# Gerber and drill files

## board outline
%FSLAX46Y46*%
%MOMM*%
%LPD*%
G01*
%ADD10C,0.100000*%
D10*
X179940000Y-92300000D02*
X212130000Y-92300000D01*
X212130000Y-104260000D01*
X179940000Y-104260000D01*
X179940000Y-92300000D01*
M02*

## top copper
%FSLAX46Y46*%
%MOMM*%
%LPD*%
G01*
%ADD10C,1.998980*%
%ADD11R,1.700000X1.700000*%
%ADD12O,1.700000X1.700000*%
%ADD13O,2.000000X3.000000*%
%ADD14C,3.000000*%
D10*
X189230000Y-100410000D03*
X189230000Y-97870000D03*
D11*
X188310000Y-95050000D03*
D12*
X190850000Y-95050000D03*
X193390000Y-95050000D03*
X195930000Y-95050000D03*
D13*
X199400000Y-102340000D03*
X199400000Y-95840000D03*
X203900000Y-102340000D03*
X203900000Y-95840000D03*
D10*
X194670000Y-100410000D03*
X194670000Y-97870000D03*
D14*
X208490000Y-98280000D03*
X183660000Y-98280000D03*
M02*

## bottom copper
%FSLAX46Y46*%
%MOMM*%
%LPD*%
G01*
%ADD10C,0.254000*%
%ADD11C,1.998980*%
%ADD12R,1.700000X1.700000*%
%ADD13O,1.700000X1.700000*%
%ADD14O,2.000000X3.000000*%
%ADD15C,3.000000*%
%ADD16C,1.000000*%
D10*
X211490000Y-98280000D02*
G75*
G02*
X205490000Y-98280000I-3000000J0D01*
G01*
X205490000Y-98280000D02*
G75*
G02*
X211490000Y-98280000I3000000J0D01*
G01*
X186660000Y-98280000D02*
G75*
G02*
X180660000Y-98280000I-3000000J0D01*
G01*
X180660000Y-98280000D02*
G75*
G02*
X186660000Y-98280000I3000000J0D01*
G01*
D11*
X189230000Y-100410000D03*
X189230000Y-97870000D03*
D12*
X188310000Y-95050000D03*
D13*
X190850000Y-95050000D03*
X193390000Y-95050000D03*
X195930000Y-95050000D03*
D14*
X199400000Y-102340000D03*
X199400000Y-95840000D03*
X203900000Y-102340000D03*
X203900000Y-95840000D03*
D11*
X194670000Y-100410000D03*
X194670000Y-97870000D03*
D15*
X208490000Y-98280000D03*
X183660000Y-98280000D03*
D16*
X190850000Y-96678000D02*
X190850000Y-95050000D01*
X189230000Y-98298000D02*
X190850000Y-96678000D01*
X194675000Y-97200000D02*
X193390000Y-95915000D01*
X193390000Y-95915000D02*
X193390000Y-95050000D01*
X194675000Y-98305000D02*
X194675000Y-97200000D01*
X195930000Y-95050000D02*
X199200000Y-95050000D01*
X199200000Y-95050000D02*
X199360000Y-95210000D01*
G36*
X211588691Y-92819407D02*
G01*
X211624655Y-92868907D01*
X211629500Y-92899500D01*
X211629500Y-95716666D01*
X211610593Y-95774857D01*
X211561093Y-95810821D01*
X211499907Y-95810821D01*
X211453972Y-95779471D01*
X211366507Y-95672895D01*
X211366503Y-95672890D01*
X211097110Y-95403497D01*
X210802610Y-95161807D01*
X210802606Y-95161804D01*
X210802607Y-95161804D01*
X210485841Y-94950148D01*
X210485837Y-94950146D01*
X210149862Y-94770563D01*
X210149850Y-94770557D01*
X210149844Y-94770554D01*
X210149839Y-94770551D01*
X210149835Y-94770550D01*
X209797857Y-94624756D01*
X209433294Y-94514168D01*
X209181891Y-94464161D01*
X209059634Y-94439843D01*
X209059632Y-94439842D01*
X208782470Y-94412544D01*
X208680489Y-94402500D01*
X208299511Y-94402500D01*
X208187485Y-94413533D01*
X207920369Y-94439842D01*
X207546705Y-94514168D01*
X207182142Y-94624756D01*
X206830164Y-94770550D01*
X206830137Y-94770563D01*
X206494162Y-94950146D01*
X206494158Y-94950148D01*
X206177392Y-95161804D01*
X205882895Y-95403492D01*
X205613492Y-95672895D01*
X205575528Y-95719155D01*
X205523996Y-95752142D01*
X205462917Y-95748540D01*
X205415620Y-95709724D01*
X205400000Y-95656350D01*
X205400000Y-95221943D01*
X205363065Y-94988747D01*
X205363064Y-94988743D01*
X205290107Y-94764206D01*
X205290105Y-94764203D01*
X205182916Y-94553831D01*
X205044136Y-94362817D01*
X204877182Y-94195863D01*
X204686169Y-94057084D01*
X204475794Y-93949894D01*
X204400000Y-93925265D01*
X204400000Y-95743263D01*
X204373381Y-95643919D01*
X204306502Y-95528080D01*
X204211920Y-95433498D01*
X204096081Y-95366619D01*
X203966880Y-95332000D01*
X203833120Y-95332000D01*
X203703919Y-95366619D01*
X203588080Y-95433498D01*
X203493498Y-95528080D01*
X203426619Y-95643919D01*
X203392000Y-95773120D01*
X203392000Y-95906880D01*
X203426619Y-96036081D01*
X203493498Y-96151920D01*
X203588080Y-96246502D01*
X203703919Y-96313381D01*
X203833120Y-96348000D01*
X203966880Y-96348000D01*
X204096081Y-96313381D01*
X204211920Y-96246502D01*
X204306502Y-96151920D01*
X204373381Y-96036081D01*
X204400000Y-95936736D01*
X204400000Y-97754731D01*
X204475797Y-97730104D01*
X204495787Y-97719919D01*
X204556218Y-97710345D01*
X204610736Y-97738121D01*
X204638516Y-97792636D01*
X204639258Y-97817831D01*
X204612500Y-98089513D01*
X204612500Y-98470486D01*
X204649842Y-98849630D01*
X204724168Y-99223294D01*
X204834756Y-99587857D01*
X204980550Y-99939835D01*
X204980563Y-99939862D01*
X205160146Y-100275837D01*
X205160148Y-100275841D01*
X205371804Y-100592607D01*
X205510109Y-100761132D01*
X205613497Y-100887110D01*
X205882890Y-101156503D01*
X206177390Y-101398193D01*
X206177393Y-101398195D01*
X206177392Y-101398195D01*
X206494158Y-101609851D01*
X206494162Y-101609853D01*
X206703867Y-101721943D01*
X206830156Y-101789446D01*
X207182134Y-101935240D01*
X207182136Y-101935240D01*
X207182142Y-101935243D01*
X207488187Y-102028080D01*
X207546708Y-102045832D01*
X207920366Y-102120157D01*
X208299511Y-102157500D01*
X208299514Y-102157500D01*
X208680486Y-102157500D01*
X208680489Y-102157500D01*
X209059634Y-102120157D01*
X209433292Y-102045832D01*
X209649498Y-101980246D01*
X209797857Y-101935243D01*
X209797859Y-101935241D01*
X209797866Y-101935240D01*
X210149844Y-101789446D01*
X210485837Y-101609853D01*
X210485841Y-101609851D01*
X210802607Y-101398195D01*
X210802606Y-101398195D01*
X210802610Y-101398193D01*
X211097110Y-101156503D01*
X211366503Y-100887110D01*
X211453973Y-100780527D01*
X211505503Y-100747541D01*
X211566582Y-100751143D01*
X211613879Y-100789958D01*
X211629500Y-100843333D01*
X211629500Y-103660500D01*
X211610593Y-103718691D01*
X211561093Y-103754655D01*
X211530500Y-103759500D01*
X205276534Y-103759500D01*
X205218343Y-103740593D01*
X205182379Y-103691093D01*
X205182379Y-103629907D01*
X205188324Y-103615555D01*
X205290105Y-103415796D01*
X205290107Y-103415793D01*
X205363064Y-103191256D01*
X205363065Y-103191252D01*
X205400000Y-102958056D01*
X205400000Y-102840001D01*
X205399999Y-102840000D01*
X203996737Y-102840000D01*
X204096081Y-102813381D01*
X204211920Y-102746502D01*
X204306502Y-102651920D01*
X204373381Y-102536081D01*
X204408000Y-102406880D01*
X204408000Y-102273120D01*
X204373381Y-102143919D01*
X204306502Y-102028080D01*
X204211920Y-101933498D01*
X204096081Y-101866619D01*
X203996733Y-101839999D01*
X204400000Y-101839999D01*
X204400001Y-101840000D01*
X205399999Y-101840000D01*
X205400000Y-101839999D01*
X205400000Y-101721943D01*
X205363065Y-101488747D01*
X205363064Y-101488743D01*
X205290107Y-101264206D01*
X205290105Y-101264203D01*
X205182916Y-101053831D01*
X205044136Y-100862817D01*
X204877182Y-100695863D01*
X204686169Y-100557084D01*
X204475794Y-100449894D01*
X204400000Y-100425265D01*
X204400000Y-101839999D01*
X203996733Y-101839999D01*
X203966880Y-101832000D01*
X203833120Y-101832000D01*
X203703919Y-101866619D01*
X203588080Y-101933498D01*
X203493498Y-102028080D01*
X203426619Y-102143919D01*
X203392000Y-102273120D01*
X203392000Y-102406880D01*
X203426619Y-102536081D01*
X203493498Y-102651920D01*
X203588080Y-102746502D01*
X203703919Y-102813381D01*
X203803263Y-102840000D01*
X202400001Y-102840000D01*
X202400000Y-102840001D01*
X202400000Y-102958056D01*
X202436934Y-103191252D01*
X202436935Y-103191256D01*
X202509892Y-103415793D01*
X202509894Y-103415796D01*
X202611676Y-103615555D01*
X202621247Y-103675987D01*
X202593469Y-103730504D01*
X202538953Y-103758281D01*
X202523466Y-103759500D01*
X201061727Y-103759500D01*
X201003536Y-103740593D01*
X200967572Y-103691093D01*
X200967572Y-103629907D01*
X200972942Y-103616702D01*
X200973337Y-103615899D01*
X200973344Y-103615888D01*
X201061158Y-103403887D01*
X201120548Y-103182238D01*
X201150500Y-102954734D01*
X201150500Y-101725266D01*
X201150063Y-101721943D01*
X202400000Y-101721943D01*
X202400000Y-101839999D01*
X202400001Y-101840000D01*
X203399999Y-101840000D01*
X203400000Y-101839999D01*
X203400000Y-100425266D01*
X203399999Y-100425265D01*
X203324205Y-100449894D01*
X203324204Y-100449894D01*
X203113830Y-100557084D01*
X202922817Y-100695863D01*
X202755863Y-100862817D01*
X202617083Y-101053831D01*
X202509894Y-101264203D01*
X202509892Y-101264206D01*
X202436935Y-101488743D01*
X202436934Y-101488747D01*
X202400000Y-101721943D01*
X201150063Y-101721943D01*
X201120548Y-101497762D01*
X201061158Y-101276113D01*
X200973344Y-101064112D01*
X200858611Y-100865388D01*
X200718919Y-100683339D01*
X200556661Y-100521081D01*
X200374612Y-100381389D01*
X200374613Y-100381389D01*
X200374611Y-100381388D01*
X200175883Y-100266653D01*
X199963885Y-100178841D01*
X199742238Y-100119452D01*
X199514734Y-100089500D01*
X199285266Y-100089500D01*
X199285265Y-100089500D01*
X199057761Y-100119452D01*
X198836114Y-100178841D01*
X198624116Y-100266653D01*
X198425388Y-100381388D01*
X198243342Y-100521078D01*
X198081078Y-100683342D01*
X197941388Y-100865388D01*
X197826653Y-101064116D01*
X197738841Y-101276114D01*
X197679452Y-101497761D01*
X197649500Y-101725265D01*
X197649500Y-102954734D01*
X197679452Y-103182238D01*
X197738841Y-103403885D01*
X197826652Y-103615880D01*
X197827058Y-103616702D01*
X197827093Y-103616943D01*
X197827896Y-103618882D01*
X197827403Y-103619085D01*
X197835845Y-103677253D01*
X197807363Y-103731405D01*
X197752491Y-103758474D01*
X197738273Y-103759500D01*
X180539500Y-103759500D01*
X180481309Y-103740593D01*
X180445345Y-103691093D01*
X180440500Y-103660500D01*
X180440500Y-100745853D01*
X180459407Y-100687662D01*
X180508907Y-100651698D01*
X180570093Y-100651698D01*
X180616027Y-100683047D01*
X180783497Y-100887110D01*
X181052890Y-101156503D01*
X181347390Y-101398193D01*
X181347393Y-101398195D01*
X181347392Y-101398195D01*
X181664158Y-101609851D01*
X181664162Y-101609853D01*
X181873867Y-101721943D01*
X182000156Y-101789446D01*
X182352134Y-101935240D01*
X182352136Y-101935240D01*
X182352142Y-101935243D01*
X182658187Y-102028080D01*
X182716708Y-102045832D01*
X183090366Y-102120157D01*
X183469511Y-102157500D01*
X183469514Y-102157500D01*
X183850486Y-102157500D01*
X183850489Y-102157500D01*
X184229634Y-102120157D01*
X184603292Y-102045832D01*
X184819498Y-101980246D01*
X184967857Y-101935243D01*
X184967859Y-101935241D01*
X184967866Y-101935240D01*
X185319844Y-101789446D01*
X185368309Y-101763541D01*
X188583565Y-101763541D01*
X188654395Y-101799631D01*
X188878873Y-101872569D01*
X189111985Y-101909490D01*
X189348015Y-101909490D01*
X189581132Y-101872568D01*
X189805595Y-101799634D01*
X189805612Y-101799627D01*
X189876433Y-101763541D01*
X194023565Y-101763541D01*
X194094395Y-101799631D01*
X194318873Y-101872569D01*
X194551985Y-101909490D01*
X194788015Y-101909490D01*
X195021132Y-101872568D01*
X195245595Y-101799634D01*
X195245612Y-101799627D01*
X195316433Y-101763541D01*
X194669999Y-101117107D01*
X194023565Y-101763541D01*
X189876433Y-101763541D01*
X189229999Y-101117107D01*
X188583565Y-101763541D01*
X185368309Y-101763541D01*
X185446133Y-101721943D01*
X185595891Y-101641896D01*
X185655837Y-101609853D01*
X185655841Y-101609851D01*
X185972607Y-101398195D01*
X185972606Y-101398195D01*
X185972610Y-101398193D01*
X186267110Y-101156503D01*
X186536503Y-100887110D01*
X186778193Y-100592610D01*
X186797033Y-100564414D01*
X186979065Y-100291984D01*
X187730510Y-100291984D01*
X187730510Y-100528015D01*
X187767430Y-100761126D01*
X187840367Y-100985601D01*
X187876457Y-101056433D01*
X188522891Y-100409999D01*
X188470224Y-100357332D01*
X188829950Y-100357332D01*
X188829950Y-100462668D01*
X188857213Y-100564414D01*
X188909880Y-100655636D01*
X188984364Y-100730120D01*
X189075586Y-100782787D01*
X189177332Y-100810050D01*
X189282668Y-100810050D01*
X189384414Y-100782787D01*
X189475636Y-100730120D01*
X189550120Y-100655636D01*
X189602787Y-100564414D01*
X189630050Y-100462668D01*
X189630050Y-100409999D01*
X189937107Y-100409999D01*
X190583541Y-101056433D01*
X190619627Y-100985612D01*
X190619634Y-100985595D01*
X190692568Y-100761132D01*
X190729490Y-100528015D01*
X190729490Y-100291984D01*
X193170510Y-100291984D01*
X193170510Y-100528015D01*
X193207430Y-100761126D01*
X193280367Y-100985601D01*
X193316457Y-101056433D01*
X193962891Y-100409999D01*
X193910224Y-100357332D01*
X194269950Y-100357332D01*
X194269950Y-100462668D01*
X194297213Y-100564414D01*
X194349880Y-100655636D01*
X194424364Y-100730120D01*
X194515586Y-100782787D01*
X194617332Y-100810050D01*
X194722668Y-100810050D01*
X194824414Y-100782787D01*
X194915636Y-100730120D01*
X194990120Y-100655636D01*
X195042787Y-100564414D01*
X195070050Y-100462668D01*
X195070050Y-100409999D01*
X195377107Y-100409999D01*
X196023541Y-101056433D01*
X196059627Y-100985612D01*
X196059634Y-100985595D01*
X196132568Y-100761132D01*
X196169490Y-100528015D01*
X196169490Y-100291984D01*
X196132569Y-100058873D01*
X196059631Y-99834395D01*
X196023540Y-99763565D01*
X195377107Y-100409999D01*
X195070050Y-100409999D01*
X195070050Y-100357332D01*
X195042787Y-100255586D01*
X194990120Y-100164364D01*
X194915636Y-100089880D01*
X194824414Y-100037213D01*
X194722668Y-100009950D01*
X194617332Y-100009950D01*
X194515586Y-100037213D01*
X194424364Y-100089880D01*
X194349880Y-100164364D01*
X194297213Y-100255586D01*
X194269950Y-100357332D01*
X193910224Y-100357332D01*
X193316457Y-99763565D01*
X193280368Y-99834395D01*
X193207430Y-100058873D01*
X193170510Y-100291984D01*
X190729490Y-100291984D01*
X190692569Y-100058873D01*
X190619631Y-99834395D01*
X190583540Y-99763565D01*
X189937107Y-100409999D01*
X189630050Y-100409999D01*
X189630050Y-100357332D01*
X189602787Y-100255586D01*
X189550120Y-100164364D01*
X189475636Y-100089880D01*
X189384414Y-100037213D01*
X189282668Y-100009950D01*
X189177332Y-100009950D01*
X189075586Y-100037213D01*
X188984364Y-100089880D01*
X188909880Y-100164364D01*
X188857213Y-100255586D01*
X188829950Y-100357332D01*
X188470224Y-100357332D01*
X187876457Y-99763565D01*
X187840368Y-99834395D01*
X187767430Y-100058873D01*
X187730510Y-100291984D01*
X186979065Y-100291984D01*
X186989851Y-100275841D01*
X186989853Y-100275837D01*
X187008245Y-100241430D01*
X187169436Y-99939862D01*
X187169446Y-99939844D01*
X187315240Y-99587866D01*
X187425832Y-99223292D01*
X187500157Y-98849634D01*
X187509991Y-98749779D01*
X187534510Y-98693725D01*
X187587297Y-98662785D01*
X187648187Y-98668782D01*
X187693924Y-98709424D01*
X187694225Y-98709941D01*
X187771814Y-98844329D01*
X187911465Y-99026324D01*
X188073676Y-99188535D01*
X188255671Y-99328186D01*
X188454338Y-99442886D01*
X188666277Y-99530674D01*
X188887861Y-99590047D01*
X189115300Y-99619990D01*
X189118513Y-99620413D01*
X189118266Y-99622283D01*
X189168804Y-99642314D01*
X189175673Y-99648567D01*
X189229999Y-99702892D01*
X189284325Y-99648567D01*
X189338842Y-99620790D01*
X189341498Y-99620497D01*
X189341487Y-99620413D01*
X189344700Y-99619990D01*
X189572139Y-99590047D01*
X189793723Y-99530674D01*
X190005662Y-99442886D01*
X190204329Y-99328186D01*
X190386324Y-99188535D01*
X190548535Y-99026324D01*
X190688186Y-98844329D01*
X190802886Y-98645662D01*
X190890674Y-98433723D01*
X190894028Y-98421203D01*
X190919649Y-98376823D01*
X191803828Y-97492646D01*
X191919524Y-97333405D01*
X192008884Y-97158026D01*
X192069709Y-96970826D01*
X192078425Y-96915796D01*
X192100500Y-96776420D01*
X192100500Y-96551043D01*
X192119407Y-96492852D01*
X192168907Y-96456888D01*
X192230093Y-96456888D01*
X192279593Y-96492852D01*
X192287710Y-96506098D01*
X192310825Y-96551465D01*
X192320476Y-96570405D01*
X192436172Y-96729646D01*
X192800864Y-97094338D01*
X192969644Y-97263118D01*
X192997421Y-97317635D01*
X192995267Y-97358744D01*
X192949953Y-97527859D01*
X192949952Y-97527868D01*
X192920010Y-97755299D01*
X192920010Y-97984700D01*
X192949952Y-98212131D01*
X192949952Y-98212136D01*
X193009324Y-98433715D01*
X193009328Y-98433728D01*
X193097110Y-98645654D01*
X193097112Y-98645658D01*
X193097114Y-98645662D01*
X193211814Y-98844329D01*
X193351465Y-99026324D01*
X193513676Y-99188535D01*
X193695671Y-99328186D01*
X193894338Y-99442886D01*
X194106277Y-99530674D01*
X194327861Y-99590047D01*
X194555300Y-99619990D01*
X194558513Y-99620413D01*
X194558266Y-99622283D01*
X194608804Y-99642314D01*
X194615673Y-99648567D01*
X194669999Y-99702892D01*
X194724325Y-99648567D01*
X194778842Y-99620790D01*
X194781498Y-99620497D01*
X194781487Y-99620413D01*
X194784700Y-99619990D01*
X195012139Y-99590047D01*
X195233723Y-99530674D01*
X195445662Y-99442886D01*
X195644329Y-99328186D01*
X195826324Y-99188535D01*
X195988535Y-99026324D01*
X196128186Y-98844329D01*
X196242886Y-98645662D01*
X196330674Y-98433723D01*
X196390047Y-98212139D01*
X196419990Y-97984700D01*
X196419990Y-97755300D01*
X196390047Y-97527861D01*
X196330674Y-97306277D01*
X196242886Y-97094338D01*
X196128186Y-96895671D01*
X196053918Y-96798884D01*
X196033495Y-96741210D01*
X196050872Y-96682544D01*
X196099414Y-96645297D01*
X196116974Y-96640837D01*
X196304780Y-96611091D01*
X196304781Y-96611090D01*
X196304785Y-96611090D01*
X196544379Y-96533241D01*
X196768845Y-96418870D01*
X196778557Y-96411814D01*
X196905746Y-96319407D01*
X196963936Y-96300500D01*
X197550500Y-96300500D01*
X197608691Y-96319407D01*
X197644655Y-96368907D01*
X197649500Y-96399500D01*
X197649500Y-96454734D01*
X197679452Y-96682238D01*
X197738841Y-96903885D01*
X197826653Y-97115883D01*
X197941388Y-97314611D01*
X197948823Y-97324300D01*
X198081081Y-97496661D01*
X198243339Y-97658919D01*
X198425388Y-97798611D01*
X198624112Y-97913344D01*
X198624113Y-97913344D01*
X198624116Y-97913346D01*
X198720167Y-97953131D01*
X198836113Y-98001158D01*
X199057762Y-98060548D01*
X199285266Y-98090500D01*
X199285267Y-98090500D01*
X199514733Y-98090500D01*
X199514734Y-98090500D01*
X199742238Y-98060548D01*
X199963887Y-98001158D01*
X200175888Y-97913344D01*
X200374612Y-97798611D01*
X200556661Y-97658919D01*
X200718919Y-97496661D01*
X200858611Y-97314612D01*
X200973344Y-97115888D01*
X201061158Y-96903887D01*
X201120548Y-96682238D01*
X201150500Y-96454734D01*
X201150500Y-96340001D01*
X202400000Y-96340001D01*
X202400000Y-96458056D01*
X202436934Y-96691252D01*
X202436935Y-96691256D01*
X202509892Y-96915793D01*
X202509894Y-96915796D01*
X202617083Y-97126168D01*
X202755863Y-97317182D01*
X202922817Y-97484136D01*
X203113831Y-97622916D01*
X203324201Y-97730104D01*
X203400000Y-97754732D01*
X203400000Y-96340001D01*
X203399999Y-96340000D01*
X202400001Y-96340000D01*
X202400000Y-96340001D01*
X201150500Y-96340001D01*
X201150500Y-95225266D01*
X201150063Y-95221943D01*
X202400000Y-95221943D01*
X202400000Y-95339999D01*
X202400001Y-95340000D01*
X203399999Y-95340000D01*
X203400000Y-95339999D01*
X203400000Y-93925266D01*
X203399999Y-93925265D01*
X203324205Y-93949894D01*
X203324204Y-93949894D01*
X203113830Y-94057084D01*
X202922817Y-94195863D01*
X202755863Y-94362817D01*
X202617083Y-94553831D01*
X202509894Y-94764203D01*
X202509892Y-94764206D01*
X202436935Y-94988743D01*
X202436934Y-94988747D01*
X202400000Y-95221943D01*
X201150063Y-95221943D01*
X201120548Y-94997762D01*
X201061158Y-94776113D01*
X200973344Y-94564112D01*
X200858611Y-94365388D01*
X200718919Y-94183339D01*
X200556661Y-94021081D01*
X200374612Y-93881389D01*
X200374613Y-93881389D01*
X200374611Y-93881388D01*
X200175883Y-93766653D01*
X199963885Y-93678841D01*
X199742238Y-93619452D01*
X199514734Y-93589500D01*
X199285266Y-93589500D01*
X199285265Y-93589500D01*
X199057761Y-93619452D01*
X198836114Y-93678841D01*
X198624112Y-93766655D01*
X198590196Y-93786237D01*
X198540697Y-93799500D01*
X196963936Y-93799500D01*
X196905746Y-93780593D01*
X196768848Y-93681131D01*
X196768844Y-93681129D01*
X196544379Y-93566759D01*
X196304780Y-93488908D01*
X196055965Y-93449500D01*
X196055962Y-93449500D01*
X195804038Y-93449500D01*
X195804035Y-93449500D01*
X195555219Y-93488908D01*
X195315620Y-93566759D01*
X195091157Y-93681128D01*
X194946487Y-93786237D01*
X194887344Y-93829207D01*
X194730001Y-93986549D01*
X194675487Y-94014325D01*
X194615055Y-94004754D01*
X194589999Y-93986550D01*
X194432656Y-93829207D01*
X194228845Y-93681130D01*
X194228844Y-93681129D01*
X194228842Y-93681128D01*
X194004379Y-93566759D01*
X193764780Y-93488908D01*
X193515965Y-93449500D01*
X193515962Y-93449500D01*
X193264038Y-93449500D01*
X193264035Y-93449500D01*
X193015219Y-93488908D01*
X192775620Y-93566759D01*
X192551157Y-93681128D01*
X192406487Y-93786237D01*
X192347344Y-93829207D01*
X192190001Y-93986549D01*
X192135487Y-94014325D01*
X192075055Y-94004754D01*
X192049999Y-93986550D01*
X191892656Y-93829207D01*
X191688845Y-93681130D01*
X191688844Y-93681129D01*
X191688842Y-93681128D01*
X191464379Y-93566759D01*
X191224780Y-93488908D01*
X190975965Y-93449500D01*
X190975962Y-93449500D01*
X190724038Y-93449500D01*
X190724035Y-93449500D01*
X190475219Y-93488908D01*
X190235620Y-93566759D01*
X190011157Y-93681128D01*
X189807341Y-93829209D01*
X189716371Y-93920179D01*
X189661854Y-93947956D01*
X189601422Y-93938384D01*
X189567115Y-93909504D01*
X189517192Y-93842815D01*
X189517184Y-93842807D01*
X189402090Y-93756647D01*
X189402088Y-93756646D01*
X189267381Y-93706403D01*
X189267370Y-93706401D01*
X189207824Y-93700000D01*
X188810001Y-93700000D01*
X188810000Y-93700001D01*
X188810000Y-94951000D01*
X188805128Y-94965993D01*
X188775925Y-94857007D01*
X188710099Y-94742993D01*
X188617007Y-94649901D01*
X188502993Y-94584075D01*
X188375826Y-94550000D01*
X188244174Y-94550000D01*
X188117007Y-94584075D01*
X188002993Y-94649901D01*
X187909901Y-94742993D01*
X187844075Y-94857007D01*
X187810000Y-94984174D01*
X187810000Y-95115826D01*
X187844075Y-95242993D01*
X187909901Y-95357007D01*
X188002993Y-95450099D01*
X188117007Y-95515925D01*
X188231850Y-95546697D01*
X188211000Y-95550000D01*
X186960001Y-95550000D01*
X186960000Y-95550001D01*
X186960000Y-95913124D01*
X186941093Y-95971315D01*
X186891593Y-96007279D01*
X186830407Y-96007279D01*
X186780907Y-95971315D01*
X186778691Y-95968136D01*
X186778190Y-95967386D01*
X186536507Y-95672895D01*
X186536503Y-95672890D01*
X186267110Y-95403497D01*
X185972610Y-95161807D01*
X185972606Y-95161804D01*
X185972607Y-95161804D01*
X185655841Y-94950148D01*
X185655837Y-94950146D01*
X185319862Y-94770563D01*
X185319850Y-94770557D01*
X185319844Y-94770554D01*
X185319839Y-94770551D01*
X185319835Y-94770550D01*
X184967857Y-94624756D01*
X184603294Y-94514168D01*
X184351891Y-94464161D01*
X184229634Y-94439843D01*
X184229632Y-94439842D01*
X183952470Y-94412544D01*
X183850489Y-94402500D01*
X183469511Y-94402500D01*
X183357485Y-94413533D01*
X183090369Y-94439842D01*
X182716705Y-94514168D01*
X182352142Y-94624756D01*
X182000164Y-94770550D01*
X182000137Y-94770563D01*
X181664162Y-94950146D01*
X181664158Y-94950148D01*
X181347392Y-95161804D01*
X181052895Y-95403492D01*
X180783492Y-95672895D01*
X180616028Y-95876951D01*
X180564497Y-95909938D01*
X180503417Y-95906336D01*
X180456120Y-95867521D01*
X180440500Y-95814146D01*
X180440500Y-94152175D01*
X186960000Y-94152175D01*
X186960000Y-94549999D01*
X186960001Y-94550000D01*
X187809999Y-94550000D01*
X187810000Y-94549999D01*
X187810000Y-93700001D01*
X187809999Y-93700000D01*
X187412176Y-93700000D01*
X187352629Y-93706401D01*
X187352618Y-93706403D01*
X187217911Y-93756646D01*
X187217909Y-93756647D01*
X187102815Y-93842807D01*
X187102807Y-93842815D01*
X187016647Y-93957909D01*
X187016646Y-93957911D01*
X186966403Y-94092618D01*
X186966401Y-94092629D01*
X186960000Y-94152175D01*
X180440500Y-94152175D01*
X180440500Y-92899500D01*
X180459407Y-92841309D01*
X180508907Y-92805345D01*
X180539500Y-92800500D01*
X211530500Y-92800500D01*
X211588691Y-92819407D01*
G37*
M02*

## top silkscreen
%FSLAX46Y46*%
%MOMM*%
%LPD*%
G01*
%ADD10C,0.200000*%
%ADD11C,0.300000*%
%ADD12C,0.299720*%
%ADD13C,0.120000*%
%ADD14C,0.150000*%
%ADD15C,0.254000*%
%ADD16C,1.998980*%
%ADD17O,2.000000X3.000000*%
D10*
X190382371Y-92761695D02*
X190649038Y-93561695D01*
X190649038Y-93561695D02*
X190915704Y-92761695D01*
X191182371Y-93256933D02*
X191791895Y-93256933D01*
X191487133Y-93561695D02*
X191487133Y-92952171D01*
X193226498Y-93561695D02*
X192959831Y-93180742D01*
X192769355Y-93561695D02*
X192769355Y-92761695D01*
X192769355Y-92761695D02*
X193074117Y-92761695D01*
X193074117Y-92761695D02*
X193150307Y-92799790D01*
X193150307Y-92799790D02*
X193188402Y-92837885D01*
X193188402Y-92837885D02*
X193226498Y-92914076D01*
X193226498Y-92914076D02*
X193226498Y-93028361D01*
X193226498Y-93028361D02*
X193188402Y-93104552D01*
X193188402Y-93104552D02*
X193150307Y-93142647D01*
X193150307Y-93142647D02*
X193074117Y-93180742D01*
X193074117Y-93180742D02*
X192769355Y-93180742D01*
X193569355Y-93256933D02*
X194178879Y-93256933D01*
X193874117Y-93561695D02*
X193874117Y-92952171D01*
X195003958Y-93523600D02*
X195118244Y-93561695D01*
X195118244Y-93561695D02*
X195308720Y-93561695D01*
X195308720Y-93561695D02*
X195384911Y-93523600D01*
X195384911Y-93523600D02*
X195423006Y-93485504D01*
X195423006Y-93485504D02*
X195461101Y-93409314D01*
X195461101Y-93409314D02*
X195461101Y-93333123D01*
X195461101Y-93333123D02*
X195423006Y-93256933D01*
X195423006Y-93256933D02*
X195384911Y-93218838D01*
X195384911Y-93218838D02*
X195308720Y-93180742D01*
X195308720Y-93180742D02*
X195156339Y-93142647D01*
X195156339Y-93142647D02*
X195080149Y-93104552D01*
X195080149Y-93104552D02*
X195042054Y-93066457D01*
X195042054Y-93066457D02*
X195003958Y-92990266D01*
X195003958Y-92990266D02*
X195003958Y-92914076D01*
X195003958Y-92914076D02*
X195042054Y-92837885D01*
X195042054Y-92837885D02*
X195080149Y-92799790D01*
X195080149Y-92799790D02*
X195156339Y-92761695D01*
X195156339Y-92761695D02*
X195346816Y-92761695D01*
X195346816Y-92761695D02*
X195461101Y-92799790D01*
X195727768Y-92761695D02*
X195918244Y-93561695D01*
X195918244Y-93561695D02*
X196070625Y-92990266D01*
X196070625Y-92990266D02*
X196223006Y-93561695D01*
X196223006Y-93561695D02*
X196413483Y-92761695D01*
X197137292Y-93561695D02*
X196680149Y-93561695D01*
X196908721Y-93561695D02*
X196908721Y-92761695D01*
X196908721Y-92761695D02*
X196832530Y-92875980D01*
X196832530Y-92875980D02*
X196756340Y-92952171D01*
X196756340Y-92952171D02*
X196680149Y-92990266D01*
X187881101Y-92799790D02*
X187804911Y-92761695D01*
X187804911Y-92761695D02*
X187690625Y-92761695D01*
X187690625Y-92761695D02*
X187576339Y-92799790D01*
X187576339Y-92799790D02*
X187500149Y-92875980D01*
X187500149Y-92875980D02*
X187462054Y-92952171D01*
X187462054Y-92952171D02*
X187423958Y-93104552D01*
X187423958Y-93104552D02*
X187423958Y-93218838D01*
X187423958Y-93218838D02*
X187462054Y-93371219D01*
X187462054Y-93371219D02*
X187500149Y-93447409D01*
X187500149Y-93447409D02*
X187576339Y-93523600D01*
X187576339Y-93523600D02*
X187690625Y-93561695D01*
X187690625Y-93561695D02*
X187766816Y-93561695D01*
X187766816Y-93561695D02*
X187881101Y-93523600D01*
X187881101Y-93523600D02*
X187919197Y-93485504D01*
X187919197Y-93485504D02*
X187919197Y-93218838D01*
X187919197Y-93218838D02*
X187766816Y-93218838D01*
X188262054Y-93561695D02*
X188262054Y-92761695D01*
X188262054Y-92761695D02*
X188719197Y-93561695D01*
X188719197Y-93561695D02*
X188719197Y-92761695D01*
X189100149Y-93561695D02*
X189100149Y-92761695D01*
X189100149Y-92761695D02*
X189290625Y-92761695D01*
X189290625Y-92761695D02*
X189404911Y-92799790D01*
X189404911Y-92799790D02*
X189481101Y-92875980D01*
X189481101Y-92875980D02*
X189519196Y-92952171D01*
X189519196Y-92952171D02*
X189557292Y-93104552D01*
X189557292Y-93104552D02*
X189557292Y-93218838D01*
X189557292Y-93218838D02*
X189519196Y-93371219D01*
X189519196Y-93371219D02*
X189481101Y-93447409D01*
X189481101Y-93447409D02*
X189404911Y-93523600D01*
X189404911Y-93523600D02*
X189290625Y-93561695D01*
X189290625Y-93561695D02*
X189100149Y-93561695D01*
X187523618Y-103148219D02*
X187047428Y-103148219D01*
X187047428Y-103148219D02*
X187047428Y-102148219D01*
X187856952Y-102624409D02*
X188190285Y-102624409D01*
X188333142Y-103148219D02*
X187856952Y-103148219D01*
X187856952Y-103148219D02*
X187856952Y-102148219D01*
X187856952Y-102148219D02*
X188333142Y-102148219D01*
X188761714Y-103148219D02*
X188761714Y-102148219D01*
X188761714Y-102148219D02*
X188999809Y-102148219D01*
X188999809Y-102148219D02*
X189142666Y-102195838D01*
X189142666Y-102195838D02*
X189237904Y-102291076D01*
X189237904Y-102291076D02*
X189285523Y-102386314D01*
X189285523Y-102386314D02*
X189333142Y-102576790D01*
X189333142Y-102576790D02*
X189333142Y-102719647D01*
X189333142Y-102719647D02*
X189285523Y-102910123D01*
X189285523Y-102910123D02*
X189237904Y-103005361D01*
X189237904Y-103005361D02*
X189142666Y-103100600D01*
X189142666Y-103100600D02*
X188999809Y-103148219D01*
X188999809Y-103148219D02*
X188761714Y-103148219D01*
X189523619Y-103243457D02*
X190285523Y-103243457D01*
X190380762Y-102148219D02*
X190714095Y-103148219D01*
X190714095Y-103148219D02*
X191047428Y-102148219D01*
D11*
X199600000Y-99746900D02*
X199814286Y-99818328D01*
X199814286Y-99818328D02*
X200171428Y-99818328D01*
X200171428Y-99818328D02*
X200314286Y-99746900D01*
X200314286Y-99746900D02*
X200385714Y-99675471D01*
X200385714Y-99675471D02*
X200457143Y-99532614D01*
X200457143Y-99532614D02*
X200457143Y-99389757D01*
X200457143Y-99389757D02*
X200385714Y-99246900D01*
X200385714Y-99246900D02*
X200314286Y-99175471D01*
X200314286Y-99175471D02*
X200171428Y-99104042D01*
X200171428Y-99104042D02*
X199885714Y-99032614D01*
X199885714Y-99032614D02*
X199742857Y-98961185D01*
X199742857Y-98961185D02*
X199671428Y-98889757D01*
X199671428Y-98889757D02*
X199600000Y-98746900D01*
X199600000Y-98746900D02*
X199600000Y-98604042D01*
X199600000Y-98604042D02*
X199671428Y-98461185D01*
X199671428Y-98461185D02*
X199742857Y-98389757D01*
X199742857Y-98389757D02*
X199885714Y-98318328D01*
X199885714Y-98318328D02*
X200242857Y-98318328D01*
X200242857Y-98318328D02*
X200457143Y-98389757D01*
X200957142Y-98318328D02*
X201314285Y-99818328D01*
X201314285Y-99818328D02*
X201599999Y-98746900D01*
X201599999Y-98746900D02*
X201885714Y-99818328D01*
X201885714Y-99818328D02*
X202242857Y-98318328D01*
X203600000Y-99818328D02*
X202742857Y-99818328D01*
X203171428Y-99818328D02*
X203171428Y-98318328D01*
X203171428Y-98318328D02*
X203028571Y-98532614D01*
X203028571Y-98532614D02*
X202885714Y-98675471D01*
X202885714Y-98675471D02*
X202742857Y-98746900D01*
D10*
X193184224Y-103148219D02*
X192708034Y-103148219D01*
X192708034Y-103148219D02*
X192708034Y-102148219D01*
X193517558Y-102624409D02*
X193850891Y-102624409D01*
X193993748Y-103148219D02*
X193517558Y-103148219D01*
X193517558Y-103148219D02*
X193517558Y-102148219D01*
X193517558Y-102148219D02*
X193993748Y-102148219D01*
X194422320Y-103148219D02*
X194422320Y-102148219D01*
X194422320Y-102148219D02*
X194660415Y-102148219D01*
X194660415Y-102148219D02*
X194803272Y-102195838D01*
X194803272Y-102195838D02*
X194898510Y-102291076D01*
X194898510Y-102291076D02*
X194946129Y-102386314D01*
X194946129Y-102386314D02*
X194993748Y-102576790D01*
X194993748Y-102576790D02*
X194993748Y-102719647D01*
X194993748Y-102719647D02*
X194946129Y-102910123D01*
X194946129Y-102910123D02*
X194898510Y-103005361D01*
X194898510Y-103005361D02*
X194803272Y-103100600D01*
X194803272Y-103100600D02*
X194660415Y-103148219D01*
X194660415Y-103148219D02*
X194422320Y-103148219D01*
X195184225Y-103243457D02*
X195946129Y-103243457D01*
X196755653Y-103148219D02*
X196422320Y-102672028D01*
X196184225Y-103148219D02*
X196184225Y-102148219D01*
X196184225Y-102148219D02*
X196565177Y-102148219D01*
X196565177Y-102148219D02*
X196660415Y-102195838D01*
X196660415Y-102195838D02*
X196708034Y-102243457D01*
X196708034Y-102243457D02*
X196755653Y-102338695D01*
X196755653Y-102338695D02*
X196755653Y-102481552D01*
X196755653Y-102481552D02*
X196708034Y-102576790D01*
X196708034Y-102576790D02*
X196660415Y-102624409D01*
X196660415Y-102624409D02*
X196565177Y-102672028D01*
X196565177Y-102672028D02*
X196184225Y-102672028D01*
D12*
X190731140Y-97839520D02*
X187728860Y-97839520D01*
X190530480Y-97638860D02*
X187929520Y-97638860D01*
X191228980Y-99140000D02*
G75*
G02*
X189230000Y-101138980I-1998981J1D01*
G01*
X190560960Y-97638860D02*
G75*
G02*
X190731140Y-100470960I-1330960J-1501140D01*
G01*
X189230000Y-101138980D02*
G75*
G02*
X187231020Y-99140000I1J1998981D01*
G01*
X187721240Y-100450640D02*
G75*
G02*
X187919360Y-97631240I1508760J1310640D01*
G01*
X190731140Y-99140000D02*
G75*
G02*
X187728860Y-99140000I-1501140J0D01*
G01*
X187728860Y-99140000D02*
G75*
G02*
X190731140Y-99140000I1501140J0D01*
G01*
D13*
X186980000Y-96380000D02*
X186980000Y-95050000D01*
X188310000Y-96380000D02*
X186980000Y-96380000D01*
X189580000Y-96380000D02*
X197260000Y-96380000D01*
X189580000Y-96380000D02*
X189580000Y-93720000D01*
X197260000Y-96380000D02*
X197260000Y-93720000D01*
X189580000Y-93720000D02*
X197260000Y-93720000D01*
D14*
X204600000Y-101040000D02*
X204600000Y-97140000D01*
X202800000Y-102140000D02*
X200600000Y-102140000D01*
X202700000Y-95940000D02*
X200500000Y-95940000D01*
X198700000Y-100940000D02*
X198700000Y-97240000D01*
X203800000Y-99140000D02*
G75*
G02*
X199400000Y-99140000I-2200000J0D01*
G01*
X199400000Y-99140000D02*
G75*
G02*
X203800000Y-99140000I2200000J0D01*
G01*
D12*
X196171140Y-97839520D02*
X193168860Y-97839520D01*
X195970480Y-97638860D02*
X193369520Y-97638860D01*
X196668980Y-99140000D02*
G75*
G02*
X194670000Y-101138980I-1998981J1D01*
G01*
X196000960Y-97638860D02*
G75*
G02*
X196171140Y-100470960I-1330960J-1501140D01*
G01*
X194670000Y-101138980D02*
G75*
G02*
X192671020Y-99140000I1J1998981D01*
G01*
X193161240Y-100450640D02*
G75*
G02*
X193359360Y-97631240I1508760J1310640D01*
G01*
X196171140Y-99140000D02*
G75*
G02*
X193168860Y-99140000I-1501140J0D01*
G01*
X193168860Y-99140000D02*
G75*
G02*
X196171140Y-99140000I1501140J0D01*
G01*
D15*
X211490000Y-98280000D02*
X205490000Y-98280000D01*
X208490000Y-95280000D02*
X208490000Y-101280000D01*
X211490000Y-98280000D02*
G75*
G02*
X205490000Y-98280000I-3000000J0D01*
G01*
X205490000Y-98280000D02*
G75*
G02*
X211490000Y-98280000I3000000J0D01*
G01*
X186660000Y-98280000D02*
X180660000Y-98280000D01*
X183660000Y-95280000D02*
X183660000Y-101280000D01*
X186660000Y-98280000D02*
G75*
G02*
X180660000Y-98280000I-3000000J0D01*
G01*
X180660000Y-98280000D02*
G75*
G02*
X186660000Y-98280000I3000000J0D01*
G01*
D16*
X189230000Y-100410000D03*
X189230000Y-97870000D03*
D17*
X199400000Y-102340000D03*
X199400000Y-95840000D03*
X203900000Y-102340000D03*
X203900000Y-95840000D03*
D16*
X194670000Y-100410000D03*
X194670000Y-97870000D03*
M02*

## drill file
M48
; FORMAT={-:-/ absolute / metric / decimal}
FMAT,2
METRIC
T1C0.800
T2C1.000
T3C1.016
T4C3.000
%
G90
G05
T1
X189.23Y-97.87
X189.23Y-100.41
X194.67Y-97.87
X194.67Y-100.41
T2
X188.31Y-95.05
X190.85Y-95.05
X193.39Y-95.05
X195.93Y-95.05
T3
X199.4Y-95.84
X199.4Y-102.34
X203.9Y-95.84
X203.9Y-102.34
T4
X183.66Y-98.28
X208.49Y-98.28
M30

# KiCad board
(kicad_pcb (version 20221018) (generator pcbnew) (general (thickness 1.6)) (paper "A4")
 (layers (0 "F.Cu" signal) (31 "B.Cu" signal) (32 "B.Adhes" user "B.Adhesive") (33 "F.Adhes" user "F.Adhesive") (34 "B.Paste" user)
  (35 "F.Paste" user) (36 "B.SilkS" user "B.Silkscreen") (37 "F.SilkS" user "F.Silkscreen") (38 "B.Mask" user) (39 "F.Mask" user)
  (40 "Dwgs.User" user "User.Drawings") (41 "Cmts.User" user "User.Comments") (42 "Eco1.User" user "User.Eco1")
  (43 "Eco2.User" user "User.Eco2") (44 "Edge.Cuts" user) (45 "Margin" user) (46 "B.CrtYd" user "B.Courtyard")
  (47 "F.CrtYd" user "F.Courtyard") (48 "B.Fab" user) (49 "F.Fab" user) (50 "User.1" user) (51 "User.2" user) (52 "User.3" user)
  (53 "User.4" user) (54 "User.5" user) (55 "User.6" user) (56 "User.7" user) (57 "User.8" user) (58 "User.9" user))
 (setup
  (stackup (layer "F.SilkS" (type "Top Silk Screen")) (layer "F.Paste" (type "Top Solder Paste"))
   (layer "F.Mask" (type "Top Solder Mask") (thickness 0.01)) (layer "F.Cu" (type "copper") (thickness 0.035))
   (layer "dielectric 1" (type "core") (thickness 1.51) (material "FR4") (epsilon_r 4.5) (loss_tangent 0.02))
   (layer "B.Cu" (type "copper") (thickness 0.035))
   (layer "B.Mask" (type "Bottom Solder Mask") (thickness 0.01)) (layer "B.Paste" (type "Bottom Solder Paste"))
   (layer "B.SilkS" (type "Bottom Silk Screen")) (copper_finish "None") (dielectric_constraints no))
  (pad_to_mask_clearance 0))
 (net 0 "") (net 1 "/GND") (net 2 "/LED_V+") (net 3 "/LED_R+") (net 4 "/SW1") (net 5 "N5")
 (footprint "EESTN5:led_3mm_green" (layer "F.Cu") (at 189.23 99.14 180)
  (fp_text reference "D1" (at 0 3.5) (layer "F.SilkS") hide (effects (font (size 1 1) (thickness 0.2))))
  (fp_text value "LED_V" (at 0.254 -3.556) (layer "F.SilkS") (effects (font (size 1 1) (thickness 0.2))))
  (fp_line (start -1.50114 1.30048) (end 1.50114 1.30048) (stroke (width 0.29972) (type solid)) (layer "F.SilkS"))
  (fp_line (start -1.30048 1.50114) (end 1.30048 1.50114) (stroke (width 0.29972) (type solid)) (layer "F.SilkS"))
  (fp_arc (start -1.99898 0) (mid -1.413492 -1.413492) (end 0 -1.99898) (stroke (width 0.29972) (type solid)) (layer "F.SilkS"))
  (fp_arc (start -1.33096 1.50114) (mid -2.002597 0.120335) (end -1.50114 -1.33096) (stroke (width 0.29972) (type solid)) (layer "F.SilkS"))
  (fp_arc (start 0 -1.99898) (mid 1.413492 -1.413492) (end 1.99898 0) (stroke (width 0.29972) (type solid)) (layer "F.SilkS"))
  (fp_arc (start 1.50876 -1.31064) (mid 1.993617 0.140092) (end 1.31064 1.50876) (stroke (width 0.29972) (type solid)) (layer "F.SilkS"))
  (fp_circle (center 0 0) (end -1.50114 0) (stroke (width 0.29972) (type solid)) (fill none) (layer "F.SilkS"))
  (pad "1" thru_hole circle (at 0 -1.27 180) (size 1.99898 1.99898) (drill 0.8001) (layers "*.Cu" "*.Mask" "F.SilkS") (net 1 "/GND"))
  (pad "2" thru_hole circle (at 0 1.27 180) (size 1.99898 1.99898) (drill 0.8001) (layers "*.Cu" "*.Mask" "F.SilkS") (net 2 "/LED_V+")))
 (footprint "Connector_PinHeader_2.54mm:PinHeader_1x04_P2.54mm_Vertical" (layer "F.Cu") (at 188.31 95.05 90)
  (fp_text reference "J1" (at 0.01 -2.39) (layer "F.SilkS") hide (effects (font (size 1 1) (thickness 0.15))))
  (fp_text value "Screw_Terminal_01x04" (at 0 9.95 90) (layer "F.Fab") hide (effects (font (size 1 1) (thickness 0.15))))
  (fp_line (start -1.33 -1.33) (end 0 -1.33) (stroke (width 0.12) (type solid)) (layer "F.SilkS"))
  (fp_line (start -1.33 0) (end -1.33 -1.33) (stroke (width 0.12) (type solid)) (layer "F.SilkS"))
  (fp_line (start -1.33 1.27) (end -1.33 8.95) (stroke (width 0.12) (type solid)) (layer "F.SilkS"))
  (fp_line (start -1.33 1.27) (end 1.33 1.27) (stroke (width 0.12) (type solid)) (layer "F.SilkS"))
  (fp_line (start -1.33 8.95) (end 1.33 8.95) (stroke (width 0.12) (type solid)) (layer "F.SilkS"))
  (fp_line (start 1.33 1.27) (end 1.33 8.95) (stroke (width 0.12) (type solid)) (layer "F.SilkS"))
  (pad "1" thru_hole rect (at 0 0 90) (size 1.7 1.7) (drill 1) (layers "*.Cu" "*.Mask") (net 1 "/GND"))
  (pad "2" thru_hole oval (at 0 2.54 90) (size 1.7 1.7) (drill 1) (layers "*.Cu" "*.Mask") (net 2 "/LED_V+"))
  (pad "3" thru_hole oval (at 0 5.08 90) (size 1.7 1.7) (drill 1) (layers "*.Cu" "*.Mask") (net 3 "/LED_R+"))
  (pad "4" thru_hole oval (at 0 7.62 90) (size 1.7 1.7) (drill 1) (layers "*.Cu" "*.Mask") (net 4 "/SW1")))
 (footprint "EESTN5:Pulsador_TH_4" (layer "F.Cu") (at 201.65 99.09 180)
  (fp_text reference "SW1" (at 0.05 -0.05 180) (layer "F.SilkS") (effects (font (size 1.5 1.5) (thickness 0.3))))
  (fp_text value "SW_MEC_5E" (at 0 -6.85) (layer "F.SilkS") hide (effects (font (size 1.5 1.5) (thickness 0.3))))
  (fp_line (start -2.95 -1.95) (end -2.95 1.95) (stroke (width 0.15) (type solid)) (layer "F.SilkS"))
  (fp_line (start -1.15 -3.05) (end 1.05 -3.05) (stroke (width 0.15) (type solid)) (layer "F.SilkS"))
  (fp_line (start -1.05 3.15) (end 1.15 3.15) (stroke (width 0.15) (type solid)) (layer "F.SilkS"))
  (fp_line (start 2.95 -1.85) (end 2.95 1.85) (stroke (width 0.15) (type solid)) (layer "F.SilkS"))
  (fp_circle (center 0.05 -0.05) (end 0.05 2.15) (stroke (width 0.15) (type solid)) (fill none) (layer "F.SilkS"))
  (pad "1" thru_hole oval (at 2.25 -3.25 180) (size 2 3) (drill 1.016) (layers "*.Cu" "*.Mask" "F.SilkS") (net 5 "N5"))
  (pad "2" thru_hole oval (at 2.25 3.25 180) (size 2 3) (drill 1.016) (layers "*.Cu" "*.Mask" "F.SilkS") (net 4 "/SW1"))
  (pad "3" thru_hole oval (at -2.25 -3.25 180) (size 2 3) (drill 1.016) (layers "*.Cu" "*.Mask" "F.SilkS") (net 1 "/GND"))
  (pad "4" thru_hole oval (at -2.25 3.25 180) (size 2 3) (drill 1.016) (layers "*.Cu" "*.Mask" "F.SilkS") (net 1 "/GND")))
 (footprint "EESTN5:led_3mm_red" (layer "F.Cu") (at 194.67 99.14 180)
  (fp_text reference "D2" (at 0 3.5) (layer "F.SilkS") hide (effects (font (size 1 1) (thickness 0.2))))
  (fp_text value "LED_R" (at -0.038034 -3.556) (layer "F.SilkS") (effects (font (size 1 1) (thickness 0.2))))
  (fp_line (start -1.50114 1.30048) (end 1.50114 1.30048) (stroke (width 0.29972) (type solid)) (layer "F.SilkS"))
  (fp_line (start -1.30048 1.50114) (end 1.30048 1.50114) (stroke (width 0.29972) (type solid)) (layer "F.SilkS"))
  (fp_arc (start -1.99898 0) (mid -1.413492 -1.413492) (end 0 -1.99898) (stroke (width 0.29972) (type solid)) (layer "F.SilkS"))
  (fp_arc (start -1.33096 1.50114) (mid -2.002597 0.120335) (end -1.50114 -1.33096) (stroke (width 0.29972) (type solid)) (layer "F.SilkS"))
  (fp_arc (start 0 -1.99898) (mid 1.413492 -1.413492) (end 1.99898 0) (stroke (width 0.29972) (type solid)) (layer "F.SilkS"))
  (fp_arc (start 1.50876 -1.31064) (mid 1.993617 0.140092) (end 1.31064 1.50876) (stroke (width 0.29972) (type solid)) (layer "F.SilkS"))
  (fp_circle (center 0 0) (end -1.50114 0) (stroke (width 0.29972) (type solid)) (fill none) (layer "F.SilkS"))
  (pad "1" thru_hole circle (at 0 -1.27 180) (size 1.99898 1.99898) (drill 0.8001) (layers "*.Cu" "*.Mask" "F.SilkS") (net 1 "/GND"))
  (pad "2" thru_hole circle (at 0 1.27 180) (size 1.99898 1.99898) (drill 0.8001) (layers "*.Cu" "*.Mask" "F.SilkS") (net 3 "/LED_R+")))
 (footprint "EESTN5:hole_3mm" (layer "B.Cu") (at 208.49 98.28 180)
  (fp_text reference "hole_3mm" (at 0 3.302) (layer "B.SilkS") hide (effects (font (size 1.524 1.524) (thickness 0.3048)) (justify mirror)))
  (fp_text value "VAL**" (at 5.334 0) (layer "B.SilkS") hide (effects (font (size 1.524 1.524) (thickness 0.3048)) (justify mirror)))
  (fp_circle (center 0 0) (end 3 0) (stroke (width 0.254) (type solid)) (fill none) (layer "B.Cu"))
  (fp_line (start -3 0) (end 3 0) (stroke (width 0.254) (type solid)) (layer "F.SilkS"))
  (fp_line (start 0 3) (end 0 -3) (stroke (width 0.254) (type solid)) (layer "F.SilkS"))
  (fp_circle (center 0 0) (end 3 0) (stroke (width 0.254) (type solid)) (fill none) (layer "F.SilkS"))
  (pad "1" thru_hole circle (at 0 0 180) (size 3 3) (drill 3) (layers "*.Cu" "B.SilkS")))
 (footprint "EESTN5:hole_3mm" (layer "B.Cu") (at 183.66 98.28 180)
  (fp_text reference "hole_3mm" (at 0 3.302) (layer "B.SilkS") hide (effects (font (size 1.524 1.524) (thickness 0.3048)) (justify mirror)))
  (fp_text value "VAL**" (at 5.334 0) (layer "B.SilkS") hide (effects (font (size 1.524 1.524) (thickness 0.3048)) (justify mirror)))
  (fp_circle (center 0 0) (end 3 0) (stroke (width 0.254) (type solid)) (fill none) (layer "B.Cu"))
  (fp_line (start -3 0) (end 3 0) (stroke (width 0.254) (type solid)) (layer "F.SilkS"))
  (fp_line (start 0 3) (end 0 -3) (stroke (width 0.254) (type solid)) (layer "F.SilkS"))
  (fp_circle (center 0 0) (end 3 0) (stroke (width 0.254) (type solid)) (fill none) (layer "F.SilkS"))
  (pad "1" thru_hole circle (at 0 0 180) (size 3 3) (drill 3) (layers "*.Cu" "B.SilkS")))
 (gr_rect (start 179.94 92.3) (end 212.13 104.26) (stroke (width 0.1) (type default)) (fill none) (layer "Edge.Cuts"))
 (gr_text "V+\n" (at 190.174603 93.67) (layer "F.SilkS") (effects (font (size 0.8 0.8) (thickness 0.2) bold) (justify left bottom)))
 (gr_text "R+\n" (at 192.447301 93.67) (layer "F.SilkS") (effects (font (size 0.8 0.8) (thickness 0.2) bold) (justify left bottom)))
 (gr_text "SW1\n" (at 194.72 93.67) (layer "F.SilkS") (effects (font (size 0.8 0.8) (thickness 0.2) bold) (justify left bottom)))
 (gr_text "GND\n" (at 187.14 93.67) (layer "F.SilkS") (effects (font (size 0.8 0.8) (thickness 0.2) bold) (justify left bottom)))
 (segment (start 190.85 96.678) (end 190.85 95.05) (width 1) (layer "B.Cu") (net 2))
 (segment (start 189.23 98.298) (end 190.85 96.678) (width 1) (layer "B.Cu") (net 2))
 (segment (start 194.675 97.2) (end 193.39 95.915) (width 1) (layer "B.Cu") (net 3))
 (segment (start 193.39 95.915) (end 193.39 95.05) (width 1) (layer "B.Cu") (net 3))
 (segment (start 194.675 98.305) (end 194.675 97.2) (width 1) (layer "B.Cu") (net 3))
 (segment (start 195.93 95.05) (end 199.2 95.05) (width 1) (layer "B.Cu") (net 4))
 (segment (start 199.2 95.05) (end 199.36 95.21) (width 1) (layer "B.Cu") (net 4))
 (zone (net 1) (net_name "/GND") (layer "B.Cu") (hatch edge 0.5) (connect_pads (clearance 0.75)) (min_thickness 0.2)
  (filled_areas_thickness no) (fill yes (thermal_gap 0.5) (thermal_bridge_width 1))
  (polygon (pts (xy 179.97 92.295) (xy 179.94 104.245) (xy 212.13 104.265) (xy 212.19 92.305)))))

